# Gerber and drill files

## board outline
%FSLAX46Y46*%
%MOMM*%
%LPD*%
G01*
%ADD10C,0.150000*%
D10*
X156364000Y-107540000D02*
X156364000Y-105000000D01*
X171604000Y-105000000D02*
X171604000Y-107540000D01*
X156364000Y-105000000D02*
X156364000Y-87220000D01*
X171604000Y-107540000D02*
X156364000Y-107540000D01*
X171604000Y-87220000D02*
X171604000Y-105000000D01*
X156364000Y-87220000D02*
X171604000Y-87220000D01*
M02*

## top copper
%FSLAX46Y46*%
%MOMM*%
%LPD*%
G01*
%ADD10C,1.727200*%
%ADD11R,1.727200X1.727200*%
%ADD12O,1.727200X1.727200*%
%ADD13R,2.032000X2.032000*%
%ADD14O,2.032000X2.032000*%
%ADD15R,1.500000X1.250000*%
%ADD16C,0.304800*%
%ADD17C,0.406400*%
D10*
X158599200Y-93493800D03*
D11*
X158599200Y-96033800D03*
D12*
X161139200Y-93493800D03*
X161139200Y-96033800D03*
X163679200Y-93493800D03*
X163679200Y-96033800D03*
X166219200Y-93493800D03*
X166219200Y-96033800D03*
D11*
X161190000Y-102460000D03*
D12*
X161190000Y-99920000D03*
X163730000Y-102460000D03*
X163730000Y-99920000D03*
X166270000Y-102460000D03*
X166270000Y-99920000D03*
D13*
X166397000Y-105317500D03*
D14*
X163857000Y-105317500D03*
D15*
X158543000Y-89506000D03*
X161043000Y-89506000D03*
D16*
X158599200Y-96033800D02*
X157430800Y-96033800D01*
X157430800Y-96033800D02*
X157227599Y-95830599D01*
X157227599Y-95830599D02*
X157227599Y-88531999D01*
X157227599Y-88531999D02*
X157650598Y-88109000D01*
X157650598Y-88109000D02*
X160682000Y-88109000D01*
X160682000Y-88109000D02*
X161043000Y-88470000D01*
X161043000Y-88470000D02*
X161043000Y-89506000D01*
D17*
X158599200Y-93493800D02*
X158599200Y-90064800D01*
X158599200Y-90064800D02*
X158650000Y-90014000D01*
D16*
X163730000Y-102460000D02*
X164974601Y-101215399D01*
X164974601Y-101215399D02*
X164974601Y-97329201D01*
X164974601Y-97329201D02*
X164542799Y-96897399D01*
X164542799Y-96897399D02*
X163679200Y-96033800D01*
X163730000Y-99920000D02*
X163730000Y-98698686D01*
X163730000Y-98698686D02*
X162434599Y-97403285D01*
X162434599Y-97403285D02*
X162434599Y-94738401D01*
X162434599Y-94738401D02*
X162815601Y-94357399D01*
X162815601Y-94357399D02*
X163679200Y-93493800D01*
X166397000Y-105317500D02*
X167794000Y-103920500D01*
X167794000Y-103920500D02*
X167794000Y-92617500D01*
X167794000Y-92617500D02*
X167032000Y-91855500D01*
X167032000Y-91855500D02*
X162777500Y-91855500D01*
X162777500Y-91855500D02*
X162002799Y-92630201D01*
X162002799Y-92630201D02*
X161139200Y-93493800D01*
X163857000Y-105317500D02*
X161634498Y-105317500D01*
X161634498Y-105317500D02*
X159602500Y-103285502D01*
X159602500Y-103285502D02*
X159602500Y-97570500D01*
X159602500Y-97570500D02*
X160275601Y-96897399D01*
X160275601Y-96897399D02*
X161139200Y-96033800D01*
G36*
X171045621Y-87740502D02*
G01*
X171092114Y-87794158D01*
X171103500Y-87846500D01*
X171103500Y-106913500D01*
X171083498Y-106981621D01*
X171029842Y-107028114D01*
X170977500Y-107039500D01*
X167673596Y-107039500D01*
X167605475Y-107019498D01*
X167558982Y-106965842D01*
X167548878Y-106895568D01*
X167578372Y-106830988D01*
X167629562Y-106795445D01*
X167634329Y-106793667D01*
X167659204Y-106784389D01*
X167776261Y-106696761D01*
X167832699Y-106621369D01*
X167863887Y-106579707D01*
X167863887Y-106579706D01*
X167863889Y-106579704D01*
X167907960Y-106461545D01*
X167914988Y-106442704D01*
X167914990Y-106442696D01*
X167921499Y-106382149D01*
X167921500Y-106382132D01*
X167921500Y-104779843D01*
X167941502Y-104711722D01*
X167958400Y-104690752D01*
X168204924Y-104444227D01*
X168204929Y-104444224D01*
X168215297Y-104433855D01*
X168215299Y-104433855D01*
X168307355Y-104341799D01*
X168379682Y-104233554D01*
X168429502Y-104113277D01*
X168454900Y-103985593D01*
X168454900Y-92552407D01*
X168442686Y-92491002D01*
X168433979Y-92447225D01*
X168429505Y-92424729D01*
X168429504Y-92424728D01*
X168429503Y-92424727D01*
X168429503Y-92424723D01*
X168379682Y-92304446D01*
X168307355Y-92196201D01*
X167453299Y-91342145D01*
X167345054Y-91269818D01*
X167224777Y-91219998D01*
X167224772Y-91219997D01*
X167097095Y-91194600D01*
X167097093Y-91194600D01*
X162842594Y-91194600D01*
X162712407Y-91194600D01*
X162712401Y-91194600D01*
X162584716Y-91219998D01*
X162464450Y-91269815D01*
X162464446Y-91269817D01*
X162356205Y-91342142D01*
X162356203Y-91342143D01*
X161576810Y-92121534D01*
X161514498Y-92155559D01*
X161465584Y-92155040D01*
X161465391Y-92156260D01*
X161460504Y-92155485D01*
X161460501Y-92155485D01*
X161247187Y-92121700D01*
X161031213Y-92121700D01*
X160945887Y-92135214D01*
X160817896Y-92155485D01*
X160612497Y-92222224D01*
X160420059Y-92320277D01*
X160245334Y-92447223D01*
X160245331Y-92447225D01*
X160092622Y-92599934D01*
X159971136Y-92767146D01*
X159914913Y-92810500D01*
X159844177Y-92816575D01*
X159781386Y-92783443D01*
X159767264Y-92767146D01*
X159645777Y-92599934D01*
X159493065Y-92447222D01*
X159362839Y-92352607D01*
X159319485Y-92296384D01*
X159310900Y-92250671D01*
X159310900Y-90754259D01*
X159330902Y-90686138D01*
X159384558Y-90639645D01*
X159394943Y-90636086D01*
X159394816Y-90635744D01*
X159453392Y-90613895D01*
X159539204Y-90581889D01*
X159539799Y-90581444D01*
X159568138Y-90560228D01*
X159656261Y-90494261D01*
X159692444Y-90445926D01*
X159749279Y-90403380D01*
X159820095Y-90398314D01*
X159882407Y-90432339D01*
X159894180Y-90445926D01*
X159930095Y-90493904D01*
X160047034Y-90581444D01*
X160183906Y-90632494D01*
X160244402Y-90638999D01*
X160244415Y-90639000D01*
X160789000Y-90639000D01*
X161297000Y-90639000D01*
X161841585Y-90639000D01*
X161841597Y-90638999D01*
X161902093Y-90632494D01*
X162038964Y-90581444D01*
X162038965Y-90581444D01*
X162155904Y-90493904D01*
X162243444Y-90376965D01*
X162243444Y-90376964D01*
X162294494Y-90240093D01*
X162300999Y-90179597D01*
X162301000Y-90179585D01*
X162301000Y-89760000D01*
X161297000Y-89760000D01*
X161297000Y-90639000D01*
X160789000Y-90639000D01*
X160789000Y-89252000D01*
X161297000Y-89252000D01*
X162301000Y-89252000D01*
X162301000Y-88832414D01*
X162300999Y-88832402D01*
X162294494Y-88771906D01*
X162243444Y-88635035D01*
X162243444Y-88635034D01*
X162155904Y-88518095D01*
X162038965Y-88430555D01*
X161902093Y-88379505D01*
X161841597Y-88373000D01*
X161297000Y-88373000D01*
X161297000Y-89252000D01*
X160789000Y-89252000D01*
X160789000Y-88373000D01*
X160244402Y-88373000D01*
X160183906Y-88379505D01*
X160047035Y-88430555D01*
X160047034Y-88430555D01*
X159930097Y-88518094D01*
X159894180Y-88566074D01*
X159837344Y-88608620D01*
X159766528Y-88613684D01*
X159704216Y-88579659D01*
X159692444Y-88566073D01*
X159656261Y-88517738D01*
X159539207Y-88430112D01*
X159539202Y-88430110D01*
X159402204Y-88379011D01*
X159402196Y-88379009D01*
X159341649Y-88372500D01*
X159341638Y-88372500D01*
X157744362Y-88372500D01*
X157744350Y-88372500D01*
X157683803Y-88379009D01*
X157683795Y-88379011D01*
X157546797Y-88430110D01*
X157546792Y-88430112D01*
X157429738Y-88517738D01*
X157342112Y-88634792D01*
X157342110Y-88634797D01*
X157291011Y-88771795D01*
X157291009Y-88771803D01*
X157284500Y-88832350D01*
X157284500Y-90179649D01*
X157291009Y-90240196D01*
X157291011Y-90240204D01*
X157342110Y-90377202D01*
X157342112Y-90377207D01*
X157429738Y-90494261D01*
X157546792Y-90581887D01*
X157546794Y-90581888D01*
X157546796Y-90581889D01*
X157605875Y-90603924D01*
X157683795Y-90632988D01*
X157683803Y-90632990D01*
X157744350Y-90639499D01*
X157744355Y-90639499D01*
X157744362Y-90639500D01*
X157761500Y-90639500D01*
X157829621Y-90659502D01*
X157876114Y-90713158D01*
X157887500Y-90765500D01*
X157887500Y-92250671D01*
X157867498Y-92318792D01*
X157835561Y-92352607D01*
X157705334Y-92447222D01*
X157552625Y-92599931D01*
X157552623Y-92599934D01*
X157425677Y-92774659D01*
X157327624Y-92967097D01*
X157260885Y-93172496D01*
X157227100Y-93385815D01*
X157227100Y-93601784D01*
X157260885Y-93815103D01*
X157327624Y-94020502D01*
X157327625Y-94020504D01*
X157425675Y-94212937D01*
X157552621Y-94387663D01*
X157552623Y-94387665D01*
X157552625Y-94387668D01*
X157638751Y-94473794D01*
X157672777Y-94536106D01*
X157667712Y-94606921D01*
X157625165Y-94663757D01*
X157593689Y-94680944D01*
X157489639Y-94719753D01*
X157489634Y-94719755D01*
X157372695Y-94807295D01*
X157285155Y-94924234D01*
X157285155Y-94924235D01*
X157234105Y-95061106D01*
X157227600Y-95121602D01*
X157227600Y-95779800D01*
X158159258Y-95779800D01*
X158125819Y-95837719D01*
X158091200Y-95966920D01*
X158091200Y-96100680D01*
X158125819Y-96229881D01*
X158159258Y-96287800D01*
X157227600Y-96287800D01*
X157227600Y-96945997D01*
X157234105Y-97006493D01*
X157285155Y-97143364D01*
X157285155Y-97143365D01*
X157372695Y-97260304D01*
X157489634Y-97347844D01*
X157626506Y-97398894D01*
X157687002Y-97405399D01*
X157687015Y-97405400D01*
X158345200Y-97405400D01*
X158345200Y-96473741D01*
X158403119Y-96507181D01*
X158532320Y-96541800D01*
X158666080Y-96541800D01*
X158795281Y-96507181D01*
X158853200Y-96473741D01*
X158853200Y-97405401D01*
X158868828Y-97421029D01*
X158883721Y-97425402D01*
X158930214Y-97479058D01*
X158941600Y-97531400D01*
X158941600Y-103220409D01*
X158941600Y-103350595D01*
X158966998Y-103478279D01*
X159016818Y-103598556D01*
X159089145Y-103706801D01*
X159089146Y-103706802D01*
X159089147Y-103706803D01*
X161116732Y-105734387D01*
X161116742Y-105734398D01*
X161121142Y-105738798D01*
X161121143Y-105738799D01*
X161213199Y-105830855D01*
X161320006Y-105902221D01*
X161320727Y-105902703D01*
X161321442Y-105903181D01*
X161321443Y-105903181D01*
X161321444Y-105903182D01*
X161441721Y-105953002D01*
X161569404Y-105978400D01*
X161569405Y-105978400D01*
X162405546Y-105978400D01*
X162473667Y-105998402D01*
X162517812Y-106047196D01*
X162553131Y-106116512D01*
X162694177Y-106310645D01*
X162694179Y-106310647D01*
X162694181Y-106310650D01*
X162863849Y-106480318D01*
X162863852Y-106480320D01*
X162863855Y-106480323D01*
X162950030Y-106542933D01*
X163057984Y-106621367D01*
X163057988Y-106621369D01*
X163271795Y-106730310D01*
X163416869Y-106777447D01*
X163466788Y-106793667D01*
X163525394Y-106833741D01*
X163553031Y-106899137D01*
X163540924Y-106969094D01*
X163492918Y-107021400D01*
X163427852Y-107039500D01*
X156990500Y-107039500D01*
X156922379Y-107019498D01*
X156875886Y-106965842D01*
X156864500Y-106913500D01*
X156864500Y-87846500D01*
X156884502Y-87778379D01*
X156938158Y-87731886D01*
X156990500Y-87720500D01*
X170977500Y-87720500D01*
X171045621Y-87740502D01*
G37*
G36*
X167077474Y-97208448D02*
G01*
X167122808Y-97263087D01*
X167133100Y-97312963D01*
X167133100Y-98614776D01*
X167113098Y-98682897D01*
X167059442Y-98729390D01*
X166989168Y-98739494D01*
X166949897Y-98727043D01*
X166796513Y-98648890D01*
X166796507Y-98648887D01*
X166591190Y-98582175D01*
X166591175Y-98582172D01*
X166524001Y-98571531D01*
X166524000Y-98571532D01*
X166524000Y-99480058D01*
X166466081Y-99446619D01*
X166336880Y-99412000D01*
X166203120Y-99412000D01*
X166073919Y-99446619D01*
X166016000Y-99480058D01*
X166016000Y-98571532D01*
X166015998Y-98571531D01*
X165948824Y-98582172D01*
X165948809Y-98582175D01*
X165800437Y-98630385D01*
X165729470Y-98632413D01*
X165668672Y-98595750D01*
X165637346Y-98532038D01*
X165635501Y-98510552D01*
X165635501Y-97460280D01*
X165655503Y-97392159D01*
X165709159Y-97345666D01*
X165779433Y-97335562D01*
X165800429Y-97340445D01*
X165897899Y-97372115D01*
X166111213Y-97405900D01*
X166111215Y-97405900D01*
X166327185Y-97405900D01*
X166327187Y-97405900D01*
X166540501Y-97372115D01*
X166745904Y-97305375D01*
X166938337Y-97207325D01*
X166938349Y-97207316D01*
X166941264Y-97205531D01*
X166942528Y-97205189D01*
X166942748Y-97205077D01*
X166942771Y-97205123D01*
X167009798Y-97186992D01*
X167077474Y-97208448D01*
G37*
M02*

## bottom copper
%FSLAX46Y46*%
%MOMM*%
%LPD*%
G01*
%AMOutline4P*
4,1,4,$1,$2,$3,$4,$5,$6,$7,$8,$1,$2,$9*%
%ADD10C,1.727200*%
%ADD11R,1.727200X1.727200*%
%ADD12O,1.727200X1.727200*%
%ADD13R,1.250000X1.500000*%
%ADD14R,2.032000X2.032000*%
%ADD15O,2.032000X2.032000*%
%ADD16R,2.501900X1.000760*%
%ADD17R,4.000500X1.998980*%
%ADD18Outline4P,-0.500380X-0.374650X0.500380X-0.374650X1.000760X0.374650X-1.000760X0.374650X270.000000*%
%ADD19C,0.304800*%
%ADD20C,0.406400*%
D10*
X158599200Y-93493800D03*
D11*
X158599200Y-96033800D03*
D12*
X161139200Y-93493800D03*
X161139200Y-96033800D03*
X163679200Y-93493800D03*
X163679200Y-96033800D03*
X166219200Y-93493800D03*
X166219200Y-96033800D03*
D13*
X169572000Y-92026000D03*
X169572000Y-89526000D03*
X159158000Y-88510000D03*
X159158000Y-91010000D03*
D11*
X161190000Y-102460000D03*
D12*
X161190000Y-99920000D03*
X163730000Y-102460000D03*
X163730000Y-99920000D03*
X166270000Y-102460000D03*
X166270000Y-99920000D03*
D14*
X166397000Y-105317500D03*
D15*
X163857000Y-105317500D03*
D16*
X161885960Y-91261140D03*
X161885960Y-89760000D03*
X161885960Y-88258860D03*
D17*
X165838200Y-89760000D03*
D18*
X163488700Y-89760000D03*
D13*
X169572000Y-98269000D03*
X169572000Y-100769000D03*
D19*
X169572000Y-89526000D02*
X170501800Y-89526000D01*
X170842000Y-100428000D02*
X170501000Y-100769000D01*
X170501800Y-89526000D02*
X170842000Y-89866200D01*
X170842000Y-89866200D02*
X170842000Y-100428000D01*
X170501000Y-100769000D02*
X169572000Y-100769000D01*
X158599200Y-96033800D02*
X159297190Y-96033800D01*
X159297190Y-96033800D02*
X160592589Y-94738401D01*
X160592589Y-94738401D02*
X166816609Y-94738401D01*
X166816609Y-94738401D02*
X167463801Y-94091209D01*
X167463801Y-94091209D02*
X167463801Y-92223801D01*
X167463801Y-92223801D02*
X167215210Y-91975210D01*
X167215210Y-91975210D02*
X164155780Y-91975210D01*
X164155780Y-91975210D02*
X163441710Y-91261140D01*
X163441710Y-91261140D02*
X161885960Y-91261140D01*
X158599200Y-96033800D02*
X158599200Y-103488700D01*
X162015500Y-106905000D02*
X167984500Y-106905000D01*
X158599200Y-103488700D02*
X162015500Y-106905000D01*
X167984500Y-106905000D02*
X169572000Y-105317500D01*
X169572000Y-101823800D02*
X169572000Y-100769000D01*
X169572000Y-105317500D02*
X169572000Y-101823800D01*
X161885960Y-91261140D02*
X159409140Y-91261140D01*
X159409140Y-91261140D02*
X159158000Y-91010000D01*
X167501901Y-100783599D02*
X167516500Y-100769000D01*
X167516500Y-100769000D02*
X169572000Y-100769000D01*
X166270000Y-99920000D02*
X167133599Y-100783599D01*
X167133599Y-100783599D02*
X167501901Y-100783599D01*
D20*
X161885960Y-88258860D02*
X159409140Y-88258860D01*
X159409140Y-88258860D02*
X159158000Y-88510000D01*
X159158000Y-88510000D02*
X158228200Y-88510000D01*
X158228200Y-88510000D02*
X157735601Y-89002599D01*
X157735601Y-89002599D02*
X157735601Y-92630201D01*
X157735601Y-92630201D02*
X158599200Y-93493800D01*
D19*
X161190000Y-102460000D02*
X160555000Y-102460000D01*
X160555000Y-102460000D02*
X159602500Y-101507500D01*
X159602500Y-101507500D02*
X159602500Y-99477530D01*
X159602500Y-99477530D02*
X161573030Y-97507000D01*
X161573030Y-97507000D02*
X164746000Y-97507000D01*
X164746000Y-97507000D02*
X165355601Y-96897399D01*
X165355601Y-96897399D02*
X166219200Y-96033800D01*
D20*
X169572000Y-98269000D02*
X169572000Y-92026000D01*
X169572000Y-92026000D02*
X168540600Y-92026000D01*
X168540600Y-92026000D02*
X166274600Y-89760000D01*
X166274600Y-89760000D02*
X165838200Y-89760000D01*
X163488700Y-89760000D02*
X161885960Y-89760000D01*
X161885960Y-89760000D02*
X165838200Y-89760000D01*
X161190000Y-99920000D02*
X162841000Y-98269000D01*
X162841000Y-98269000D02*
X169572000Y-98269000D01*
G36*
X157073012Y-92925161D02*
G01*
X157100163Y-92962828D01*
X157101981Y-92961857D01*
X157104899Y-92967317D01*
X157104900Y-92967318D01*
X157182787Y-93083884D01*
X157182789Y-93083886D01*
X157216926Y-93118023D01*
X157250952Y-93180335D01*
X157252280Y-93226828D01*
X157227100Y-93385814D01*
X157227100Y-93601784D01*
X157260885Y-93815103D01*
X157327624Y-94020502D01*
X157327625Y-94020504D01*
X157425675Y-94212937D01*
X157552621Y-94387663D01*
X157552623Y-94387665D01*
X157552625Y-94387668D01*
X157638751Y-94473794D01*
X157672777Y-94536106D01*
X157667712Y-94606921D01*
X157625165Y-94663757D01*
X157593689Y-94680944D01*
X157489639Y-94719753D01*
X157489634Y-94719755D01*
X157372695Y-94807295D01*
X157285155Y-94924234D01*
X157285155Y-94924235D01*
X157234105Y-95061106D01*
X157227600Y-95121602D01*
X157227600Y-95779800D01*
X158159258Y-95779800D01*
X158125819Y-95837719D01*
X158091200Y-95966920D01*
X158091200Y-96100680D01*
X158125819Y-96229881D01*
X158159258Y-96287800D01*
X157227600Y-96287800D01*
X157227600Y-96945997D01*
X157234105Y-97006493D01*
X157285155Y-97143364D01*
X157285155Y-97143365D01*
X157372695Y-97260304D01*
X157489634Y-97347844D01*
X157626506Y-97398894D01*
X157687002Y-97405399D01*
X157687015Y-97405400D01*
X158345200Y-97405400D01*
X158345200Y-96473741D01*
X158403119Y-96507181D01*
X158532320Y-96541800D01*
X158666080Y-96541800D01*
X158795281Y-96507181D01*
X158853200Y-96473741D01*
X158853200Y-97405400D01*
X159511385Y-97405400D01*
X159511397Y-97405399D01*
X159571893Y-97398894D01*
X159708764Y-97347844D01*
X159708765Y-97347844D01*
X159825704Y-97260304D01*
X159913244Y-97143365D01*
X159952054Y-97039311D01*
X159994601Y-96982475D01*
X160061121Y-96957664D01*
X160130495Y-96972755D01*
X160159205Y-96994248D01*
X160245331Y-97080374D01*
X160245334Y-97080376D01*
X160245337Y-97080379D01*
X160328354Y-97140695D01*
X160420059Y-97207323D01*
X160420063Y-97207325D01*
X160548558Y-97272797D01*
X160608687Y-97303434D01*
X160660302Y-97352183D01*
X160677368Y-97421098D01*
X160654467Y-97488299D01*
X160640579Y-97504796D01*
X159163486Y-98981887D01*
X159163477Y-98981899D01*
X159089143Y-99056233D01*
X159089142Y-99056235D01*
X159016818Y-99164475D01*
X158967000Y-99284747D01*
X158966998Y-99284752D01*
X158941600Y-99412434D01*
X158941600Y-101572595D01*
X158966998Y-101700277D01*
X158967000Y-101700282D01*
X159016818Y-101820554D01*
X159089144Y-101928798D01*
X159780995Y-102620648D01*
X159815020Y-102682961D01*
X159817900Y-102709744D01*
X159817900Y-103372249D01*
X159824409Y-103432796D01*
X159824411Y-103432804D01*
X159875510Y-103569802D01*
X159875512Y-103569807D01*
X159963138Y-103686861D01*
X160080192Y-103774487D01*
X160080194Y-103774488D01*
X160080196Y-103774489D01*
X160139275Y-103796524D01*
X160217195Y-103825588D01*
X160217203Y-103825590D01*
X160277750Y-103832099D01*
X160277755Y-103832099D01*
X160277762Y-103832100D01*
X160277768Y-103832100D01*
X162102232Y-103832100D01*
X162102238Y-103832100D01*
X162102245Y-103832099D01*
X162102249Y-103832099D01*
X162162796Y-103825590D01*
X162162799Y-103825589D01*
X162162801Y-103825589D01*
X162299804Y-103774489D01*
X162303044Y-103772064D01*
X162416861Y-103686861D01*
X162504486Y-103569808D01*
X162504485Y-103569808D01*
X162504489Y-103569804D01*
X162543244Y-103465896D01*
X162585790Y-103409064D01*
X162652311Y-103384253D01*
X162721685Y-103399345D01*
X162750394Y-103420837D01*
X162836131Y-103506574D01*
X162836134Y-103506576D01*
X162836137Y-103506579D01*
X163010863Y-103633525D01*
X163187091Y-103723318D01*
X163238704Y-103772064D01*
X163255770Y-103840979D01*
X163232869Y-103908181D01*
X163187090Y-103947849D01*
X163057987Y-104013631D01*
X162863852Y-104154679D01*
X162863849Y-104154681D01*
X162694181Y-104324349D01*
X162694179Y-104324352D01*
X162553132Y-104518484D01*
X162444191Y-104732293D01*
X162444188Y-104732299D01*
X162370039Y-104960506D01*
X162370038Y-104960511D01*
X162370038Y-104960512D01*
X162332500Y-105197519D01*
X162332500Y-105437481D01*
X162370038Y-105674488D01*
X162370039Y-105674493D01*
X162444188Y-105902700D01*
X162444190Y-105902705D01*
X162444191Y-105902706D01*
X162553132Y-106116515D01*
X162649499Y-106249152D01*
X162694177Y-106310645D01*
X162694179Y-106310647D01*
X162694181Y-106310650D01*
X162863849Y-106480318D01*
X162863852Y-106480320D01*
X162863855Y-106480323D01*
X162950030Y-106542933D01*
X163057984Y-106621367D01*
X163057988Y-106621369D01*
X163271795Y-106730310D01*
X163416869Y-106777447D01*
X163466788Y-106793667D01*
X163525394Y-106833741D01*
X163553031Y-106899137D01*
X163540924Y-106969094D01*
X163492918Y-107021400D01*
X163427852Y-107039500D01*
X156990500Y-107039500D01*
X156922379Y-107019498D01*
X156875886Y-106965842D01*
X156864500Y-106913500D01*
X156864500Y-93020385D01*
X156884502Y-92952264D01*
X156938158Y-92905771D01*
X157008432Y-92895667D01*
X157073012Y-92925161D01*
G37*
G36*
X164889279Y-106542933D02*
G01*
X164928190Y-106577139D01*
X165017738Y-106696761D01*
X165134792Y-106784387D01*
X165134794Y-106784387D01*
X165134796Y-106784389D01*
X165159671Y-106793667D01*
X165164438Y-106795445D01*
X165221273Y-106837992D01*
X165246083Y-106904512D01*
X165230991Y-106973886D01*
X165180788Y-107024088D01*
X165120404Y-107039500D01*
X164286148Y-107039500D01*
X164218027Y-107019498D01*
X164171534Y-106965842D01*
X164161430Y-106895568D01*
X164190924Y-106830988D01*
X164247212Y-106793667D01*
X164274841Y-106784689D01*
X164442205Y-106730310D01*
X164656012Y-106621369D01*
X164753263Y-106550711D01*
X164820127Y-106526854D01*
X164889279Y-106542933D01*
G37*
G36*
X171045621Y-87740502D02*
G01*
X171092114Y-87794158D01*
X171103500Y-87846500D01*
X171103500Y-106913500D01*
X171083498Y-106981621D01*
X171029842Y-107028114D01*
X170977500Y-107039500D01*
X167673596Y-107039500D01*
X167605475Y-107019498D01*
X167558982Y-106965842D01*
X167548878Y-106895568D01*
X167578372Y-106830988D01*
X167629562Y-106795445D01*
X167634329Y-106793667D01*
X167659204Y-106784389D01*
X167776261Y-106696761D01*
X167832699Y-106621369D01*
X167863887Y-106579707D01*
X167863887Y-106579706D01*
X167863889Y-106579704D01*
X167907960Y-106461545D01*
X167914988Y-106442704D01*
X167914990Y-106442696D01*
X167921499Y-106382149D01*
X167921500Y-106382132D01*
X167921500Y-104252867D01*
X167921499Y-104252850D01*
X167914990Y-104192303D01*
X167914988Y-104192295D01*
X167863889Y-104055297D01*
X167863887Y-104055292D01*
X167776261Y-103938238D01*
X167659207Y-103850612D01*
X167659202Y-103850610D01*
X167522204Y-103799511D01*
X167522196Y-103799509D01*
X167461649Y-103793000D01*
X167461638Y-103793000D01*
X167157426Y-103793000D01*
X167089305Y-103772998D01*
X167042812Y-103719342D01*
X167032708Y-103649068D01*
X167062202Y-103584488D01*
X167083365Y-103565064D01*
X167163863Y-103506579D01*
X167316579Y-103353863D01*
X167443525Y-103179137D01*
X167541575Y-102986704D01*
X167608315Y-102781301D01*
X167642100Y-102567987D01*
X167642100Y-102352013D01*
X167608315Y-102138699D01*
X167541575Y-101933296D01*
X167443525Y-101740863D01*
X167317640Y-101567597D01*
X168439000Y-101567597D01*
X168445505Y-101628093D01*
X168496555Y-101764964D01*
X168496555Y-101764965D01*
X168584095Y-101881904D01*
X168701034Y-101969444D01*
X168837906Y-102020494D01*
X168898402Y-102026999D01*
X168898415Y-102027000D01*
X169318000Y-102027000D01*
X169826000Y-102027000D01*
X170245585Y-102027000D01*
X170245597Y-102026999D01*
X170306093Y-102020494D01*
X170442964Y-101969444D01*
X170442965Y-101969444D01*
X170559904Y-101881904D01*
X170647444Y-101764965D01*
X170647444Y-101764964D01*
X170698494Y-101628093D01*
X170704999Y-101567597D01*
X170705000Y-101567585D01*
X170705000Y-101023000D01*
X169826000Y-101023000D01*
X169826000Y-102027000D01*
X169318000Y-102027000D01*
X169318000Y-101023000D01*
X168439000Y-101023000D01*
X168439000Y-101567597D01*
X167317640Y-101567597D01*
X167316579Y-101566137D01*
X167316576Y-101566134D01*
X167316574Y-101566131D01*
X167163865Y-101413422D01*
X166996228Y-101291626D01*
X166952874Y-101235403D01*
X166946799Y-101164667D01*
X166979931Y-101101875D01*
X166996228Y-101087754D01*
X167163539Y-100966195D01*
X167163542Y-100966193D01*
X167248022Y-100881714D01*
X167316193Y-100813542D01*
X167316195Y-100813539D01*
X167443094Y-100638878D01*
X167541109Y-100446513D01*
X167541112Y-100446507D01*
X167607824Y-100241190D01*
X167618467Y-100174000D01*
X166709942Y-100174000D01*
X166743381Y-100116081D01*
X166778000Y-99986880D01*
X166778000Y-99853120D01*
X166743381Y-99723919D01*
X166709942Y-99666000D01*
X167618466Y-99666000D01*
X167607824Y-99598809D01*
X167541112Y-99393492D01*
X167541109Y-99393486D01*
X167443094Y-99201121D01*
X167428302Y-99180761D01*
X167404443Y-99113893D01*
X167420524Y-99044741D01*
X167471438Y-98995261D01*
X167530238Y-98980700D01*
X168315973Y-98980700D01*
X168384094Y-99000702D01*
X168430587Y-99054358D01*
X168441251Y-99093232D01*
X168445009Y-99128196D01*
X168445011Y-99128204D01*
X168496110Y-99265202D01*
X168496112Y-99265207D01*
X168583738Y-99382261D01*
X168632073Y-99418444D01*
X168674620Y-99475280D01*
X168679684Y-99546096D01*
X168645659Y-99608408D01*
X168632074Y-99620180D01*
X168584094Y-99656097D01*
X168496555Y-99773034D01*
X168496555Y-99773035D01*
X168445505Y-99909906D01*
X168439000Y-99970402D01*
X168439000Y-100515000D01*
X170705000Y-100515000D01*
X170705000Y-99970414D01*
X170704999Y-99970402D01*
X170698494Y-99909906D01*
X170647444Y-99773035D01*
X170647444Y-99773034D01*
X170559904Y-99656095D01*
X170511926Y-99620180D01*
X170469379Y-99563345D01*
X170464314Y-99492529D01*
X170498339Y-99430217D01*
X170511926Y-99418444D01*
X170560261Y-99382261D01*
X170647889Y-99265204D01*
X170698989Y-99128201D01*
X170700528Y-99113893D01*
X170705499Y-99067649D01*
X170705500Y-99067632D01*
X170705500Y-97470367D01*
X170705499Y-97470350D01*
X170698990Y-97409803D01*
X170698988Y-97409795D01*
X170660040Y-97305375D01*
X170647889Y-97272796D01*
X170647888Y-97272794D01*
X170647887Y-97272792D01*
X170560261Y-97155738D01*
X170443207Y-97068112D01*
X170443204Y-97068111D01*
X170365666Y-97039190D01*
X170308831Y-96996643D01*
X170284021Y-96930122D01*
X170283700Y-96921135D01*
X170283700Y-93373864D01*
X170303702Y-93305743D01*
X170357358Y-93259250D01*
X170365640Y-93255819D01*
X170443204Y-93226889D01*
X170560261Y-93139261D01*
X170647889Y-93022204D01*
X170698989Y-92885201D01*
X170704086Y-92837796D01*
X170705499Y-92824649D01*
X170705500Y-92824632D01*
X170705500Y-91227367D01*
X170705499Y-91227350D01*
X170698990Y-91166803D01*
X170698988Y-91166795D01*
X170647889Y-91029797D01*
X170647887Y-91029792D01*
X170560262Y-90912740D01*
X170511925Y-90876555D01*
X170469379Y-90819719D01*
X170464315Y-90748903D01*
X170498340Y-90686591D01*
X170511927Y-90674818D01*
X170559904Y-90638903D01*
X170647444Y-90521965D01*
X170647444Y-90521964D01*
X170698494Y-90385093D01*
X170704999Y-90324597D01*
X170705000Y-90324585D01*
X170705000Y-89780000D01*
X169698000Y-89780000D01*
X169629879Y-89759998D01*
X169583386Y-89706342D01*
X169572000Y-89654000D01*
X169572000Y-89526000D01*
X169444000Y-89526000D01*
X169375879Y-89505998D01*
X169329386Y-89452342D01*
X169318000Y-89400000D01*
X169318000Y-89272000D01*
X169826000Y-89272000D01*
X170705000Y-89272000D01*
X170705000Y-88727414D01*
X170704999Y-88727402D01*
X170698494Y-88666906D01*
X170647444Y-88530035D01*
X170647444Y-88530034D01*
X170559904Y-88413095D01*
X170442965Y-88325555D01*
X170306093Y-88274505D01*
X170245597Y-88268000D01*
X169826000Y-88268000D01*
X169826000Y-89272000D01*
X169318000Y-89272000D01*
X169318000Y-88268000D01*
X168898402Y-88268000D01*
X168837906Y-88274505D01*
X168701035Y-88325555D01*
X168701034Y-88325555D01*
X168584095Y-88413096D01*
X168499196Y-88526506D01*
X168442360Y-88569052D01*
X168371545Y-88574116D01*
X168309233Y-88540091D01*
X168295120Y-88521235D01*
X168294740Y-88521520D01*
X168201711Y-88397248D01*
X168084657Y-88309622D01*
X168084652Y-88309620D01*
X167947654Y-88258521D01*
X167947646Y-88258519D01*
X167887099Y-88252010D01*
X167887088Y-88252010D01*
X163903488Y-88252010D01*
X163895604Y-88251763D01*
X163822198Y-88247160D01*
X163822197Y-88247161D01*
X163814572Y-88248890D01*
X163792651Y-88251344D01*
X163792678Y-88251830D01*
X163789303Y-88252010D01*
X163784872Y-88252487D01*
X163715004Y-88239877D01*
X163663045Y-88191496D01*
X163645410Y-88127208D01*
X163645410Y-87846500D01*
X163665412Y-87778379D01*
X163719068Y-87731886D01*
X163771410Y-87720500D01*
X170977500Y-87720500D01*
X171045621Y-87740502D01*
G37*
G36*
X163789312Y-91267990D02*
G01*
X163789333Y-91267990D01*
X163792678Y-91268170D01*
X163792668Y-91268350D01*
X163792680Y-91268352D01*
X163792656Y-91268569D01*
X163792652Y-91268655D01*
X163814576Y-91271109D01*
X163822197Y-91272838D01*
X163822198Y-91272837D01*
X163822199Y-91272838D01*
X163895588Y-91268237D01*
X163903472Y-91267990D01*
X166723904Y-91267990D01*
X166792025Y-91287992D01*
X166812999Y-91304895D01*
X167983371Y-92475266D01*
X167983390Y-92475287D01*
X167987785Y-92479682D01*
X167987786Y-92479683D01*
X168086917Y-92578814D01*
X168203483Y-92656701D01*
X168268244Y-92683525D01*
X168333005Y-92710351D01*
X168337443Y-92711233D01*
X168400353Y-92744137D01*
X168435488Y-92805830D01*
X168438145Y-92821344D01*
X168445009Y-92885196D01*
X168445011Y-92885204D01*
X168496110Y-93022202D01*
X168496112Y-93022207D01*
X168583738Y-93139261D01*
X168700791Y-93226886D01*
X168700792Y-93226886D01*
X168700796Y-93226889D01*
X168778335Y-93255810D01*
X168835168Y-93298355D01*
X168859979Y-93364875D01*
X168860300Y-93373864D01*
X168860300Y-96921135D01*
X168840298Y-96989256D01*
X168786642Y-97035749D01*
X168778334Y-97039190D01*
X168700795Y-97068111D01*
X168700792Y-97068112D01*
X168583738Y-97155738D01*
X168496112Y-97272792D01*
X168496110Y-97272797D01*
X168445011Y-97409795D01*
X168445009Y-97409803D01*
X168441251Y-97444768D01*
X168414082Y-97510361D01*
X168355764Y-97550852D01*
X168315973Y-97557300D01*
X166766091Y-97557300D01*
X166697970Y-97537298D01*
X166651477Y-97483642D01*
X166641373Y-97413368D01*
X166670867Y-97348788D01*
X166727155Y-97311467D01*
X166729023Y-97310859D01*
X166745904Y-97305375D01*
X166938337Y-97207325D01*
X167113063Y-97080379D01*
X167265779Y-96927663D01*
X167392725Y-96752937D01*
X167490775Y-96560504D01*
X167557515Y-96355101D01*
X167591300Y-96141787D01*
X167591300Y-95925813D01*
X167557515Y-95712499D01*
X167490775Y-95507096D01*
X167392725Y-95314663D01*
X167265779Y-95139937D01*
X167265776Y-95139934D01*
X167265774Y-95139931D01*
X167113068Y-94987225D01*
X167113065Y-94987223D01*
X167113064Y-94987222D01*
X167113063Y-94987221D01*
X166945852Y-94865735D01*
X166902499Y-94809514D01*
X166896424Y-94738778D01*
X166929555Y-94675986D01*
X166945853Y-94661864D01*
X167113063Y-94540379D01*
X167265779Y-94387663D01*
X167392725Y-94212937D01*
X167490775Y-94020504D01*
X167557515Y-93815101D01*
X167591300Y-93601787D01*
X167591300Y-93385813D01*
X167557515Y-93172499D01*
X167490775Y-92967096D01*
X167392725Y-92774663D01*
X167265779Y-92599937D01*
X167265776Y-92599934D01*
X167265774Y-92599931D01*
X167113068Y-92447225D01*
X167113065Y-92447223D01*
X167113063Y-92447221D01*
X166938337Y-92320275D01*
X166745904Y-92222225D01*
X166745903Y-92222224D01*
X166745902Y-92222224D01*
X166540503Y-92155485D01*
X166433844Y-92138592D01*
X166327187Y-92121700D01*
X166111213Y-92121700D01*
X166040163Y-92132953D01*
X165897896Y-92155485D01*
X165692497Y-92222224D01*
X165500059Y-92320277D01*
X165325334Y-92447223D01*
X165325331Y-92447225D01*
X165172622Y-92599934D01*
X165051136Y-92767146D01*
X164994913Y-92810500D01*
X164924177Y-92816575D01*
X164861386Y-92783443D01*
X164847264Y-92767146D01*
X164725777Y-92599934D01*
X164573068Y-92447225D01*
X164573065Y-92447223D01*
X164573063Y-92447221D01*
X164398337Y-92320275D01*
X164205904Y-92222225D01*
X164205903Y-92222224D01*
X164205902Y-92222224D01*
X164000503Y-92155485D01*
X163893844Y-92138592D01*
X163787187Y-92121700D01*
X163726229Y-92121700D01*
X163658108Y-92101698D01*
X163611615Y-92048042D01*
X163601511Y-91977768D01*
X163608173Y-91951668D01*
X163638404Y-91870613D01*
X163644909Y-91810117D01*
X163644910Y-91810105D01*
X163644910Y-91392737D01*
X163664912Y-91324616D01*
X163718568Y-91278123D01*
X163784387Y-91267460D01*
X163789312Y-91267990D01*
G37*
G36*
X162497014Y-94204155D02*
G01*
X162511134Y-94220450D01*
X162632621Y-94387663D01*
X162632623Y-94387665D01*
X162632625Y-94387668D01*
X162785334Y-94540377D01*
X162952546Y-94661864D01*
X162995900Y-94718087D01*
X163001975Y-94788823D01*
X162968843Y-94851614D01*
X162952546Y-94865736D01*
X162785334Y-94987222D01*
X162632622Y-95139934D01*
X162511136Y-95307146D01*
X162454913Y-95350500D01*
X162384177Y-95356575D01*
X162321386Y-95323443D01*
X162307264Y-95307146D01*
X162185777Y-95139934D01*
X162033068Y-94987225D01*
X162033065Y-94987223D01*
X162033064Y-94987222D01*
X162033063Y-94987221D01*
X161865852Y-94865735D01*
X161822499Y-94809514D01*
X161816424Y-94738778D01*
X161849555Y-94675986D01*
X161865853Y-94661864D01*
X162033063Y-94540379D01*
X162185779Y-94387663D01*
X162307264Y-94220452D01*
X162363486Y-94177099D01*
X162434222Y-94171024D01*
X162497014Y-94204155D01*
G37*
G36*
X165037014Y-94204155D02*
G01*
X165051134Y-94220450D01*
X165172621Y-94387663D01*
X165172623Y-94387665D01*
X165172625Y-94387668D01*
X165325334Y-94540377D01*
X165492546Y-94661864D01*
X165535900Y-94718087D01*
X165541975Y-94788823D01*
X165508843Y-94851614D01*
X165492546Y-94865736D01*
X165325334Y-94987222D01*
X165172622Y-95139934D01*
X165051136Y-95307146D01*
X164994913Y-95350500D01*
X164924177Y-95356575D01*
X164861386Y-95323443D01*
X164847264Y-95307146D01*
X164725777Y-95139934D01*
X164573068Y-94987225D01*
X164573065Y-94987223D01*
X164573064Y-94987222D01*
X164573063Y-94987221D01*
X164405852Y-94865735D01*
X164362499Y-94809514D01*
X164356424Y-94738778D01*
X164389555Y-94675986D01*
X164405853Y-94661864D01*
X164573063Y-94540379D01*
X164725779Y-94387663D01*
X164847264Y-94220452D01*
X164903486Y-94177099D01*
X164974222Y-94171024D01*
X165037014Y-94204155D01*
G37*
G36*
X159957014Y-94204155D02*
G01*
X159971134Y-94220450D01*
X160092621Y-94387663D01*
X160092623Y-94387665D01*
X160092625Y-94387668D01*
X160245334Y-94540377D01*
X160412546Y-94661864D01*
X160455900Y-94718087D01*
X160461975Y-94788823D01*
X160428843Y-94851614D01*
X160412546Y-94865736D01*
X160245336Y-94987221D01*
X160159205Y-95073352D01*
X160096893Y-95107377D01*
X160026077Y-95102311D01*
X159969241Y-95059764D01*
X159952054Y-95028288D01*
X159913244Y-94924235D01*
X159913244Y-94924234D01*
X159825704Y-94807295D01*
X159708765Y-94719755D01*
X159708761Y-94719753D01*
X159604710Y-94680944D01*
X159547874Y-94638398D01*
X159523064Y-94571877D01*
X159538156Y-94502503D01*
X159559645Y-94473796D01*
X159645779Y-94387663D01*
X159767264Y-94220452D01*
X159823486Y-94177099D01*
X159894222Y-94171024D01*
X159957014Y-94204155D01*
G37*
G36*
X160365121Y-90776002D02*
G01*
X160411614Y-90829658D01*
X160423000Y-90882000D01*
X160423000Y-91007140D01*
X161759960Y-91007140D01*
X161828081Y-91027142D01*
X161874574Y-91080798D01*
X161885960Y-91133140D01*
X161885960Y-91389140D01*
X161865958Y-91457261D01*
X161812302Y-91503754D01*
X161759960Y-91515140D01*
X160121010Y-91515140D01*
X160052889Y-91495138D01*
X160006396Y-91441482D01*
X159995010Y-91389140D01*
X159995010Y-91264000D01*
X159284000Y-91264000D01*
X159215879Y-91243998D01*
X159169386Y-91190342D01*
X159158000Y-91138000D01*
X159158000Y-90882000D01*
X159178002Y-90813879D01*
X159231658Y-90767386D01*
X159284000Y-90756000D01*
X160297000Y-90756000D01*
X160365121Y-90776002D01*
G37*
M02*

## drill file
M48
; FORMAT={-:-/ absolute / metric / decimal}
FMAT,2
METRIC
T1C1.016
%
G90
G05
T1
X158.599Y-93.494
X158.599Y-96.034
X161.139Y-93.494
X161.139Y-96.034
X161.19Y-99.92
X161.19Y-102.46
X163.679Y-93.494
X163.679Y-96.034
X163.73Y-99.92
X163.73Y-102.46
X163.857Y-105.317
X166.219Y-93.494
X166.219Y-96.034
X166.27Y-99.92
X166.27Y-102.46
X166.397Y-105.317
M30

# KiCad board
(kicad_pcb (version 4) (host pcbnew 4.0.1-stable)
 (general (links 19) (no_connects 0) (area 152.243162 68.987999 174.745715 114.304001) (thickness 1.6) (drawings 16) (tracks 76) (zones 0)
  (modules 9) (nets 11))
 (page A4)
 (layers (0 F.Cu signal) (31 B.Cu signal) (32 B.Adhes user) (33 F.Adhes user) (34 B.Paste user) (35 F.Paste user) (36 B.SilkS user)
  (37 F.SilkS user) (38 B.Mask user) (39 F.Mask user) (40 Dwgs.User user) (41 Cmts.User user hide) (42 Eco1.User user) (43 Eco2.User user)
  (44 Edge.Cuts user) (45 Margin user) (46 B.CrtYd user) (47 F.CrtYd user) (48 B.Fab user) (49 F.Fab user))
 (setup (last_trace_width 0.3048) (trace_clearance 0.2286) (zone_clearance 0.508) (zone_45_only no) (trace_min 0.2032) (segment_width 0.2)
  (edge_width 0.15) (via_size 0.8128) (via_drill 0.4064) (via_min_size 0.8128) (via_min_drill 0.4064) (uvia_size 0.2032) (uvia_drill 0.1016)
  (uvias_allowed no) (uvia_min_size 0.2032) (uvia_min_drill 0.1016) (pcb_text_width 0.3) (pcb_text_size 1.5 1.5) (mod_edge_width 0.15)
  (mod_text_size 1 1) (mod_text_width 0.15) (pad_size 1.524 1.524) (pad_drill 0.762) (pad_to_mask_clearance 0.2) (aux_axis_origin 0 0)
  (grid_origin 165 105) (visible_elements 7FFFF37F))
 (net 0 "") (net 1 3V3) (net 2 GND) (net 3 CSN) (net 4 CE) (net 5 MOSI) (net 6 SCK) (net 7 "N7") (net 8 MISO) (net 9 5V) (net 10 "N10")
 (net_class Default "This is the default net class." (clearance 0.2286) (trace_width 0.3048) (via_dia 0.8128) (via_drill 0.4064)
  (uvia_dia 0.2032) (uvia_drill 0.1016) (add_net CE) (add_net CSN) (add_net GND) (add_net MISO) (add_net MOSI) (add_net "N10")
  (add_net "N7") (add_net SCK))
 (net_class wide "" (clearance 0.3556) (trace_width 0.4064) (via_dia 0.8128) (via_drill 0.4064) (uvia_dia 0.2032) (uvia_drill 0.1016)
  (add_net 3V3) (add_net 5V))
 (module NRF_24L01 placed (layer F.Cu) (at 162.46 93.57)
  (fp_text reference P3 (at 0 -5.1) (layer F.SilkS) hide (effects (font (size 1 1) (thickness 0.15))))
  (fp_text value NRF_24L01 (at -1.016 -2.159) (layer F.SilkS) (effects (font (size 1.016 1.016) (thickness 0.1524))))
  (pad 2 thru_hole circle (at -3.8608 -0.0762) (size 1.7272 1.7272) (drill 1.016) (layers *.Cu *.Mask F.SilkS) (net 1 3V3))
  (pad 1 thru_hole rect (at -3.8608 2.4638) (size 1.7272 1.7272) (drill 1.016) (layers *.Cu *.Mask F.SilkS) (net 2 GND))
  (pad 4 thru_hole oval (at -1.3208 -0.0762) (size 1.7272 1.7272) (drill 1.016) (layers *.Cu *.Mask F.SilkS) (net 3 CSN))
  (pad 3 thru_hole oval (at -1.3208 2.4638) (size 1.7272 1.7272) (drill 1.016) (layers *.Cu *.Mask F.SilkS) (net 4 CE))
  (pad 6 thru_hole oval (at 1.2192 -0.0762) (size 1.7272 1.7272) (drill 1.016) (layers *.Cu *.Mask F.SilkS) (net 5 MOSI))
  (pad 5 thru_hole oval (at 1.2192 2.4638) (size 1.7272 1.7272) (drill 1.016) (layers *.Cu *.Mask F.SilkS) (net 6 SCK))
  (pad 8 thru_hole oval (at 3.7592 -0.0762) (size 1.7272 1.7272) (drill 1.016) (layers *.Cu *.Mask F.SilkS) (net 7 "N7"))
  (pad 7 thru_hole oval (at 3.7592 2.4638) (size 1.7272 1.7272) (drill 1.016) (layers *.Cu *.Mask F.SilkS) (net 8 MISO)))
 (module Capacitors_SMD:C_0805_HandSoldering (layer B.Cu) (at 169.572 90.776 90)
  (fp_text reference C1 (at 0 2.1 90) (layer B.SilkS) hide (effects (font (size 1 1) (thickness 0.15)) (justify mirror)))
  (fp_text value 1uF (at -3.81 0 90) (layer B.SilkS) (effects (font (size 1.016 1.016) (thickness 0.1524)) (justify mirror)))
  (pad 1 smd rect (at -1.25 0 90) (size 1.5 1.25) (layers B.Cu B.Paste B.Mask) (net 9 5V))
  (pad 2 smd rect (at 1.25 0 90) (size 1.5 1.25) (layers B.Cu B.Paste B.Mask) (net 2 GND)))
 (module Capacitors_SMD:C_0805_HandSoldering (layer B.Cu) (at 159.158 89.76 270)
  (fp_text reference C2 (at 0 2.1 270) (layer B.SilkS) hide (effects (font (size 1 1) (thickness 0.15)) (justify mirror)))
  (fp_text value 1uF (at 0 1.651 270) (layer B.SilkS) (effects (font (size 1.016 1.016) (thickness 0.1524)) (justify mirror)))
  (pad 1 smd rect (at -1.25 0 270) (size 1.5 1.25) (layers B.Cu B.Paste B.Mask) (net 1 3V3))
  (pad 2 smd rect (at 1.25 0 270) (size 1.5 1.25) (layers B.Cu B.Paste B.Mask) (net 2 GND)))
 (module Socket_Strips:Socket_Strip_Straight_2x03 (layer B.Cu) (at 161.19 102.46)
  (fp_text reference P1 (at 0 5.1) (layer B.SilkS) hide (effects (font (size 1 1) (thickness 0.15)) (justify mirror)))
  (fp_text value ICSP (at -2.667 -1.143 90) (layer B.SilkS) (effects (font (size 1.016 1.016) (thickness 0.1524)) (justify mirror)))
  (pad 1 thru_hole rect (at 0 0) (size 1.7272 1.7272) (drill 1.016) (layers *.Cu *.Mask B.SilkS) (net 8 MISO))
  (pad 2 thru_hole oval (at 0 -2.54) (size 1.7272 1.7272) (drill 1.016) (layers *.Cu *.Mask B.SilkS) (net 9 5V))
  (pad 3 thru_hole oval (at 2.54 0) (size 1.7272 1.7272) (drill 1.016) (layers *.Cu *.Mask B.SilkS) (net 6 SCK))
  (pad 4 thru_hole oval (at 2.54 -2.54) (size 1.7272 1.7272) (drill 1.016) (layers *.Cu *.Mask B.SilkS) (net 5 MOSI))
  (pad 5 thru_hole oval (at 5.08 0) (size 1.7272 1.7272) (drill 1.016) (layers *.Cu *.Mask B.SilkS) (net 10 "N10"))
  (pad 6 thru_hole oval (at 5.08 -2.54) (size 1.7272 1.7272) (drill 1.016) (layers *.Cu *.Mask B.SilkS) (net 2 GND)))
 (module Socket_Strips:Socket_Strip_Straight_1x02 (layer F.Cu) (at 166.397 105.3175 180)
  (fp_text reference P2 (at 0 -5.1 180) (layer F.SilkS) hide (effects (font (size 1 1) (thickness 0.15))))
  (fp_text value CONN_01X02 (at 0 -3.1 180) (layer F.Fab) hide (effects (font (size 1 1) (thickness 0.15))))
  (pad 1 thru_hole rect (at 0 0 180) (size 2.032 2.032) (drill 1.016) (layers *.Cu *.Mask F.SilkS) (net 3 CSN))
  (pad 2 thru_hole oval (at 2.54 0 180) (size 2.032 2.032) (drill 1.016) (layers *.Cu *.Mask F.SilkS) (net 4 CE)))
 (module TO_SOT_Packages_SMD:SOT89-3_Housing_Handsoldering (layer B.Cu) (at 164.238 89.76 90)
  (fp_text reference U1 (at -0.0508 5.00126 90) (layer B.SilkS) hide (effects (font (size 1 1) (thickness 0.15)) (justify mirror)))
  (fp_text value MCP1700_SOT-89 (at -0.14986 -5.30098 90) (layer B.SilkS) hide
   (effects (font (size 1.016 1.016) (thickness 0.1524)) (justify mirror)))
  (pad 1 smd rect (at -1.50114 -2.35204 90) (size 1.00076 2.5019) (layers B.Cu B.Paste B.Mask) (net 2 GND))
  (pad 2 smd rect (at 0 -2.35204 90) (size 1.00076 2.5019) (layers B.Cu B.Paste B.Mask) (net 9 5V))
  (pad 3 smd rect (at 1.50114 -2.35204 90) (size 1.00076 2.5019) (layers B.Cu B.Paste B.Mask) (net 1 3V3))
  (pad 2 smd rect (at 0 1.6002 90) (size 1.99898 4.0005) (layers B.Cu B.Paste B.Mask) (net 9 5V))
  (pad 2 smd trapezoid (at 0 -0.7493 270) (size 1.50114 0.7493) (rect_delta 0 -0.50038) (layers B.Cu B.Paste B.Mask) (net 9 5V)))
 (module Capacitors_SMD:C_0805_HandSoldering (layer F.Cu) (at 159.793 89.506)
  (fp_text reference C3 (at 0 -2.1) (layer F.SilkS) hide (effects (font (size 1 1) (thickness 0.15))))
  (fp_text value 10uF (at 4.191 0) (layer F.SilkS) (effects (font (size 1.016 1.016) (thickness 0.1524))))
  (pad 1 smd rect (at -1.25 0) (size 1.5 1.25) (layers F.Cu F.Paste F.Mask) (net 1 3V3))
  (pad 2 smd rect (at 1.25 0) (size 1.5 1.25) (layers F.Cu F.Paste F.Mask) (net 2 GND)))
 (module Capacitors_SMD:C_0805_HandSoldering (layer B.Cu) (at 169.572 99.519 270)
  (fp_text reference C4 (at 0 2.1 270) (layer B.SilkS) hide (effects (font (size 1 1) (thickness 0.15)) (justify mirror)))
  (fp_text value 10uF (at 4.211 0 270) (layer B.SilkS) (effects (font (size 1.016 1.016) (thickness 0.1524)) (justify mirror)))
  (pad 1 smd rect (at -1.25 0 270) (size 1.5 1.25) (layers B.Cu B.Paste B.Mask) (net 9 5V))
  (pad 2 smd rect (at 1.25 0 270) (size 1.5 1.25) (layers B.Cu B.Paste B.Mask) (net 2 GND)))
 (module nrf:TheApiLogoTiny (layer F.Cu) (at 158.269 102.206)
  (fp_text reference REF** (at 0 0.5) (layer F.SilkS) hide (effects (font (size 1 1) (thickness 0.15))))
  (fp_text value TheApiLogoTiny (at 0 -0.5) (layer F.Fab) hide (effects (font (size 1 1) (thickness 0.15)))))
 (gr_line (start 156.364 107.54) (end 156.364 105) (angle 90) (layer Edge.Cuts) (width 0.15))
 (gr_line (start 171.604 105) (end 171.604 107.54) (angle 90) (layer Edge.Cuts) (width 0.15))
 (gr_line (start 156.364 105) (end 156.364 87.22) (angle 90) (layer Edge.Cuts) (width 0.15))
 (gr_line (start 171.604 107.54) (end 156.364 107.54) (angle 90) (layer Edge.Cuts) (width 0.15))
 (gr_line (start 171.604 87.22) (end 171.604 105) (angle 90) (layer Edge.Cuts) (width 0.15))
 (gr_line (start 156.364 87.22) (end 171.604 87.22) (angle 90) (layer Edge.Cuts) (width 0.15))
 (segment (start 158.5992 96.0338) (end 157.4308 96.0338) (width 0.3048) (layer F.Cu) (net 2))
 (segment (start 157.4308 96.0338) (end 157.227599 95.830599) (width 0.3048) (layer F.Cu) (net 2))
 (segment (start 157.227599 95.830599) (end 157.227599 88.531999) (width 0.3048) (layer F.Cu) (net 2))
 (segment (start 157.227599 88.531999) (end 157.650598 88.109) (width 0.3048) (layer F.Cu) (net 2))
 (segment (start 157.650598 88.109) (end 160.682 88.109) (width 0.3048) (layer F.Cu) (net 2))
 (segment (start 160.682 88.109) (end 161.043 88.47) (width 0.3048) (layer F.Cu) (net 2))
 (segment (start 161.043 88.47) (end 161.043 89.506) (width 0.3048) (layer F.Cu) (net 2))
 (segment (start 169.572 89.526) (end 170.5018 89.526) (width 0.3048) (layer B.Cu) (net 2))
 (segment (start 170.842 100.428) (end 170.501 100.769) (width 0.3048) (layer B.Cu) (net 2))
 (segment (start 170.5018 89.526) (end 170.842 89.8662) (width 0.3048) (layer B.Cu) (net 2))
 (segment (start 170.842 89.8662) (end 170.842 100.428) (width 0.3048) (layer B.Cu) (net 2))
 (segment (start 170.501 100.769) (end 169.572 100.769) (width 0.3048) (layer B.Cu) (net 2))
 (segment (start 158.5992 96.0338) (end 159.29719 96.0338) (width 0.3048) (layer B.Cu) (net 2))
 (segment (start 159.29719 96.0338) (end 160.592589 94.738401) (width 0.3048) (layer B.Cu) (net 2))
 (segment (start 160.592589 94.738401) (end 166.816609 94.738401) (width 0.3048) (layer B.Cu) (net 2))
 (segment (start 166.816609 94.738401) (end 167.463801 94.091209) (width 0.3048) (layer B.Cu) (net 2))
 (segment (start 167.463801 94.091209) (end 167.463801 92.223801) (width 0.3048) (layer B.Cu) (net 2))
 (segment (start 167.463801 92.223801) (end 167.21521 91.97521) (width 0.3048) (layer B.Cu) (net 2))
 (segment (start 167.21521 91.97521) (end 164.15578 91.97521) (width 0.3048) (layer B.Cu) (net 2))
 (segment (start 164.15578 91.97521) (end 163.44171 91.26114) (width 0.3048) (layer B.Cu) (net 2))
 (segment (start 163.44171 91.26114) (end 161.88596 91.26114) (width 0.3048) (layer B.Cu) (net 2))
 (segment (start 158.5992 96.0338) (end 158.5992 103.4887) (width 0.3048) (layer B.Cu) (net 2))
 (segment (start 162.0155 106.905) (end 167.9845 106.905) (width 0.3048) (layer B.Cu) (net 2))
 (segment (start 158.5992 103.4887) (end 162.0155 106.905) (width 0.3048) (layer B.Cu) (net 2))
 (segment (start 167.9845 106.905) (end 169.572 105.3175) (width 0.3048) (layer B.Cu) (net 2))
 (segment (start 169.572 101.8238) (end 169.572 100.769) (width 0.3048) (layer B.Cu) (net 2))
 (segment (start 169.572 105.3175) (end 169.572 101.8238) (width 0.3048) (layer B.Cu) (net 2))
 (segment (start 161.88596 91.26114) (end 159.40914 91.26114) (width 0.3048) (layer B.Cu) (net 2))
 (segment (start 159.40914 91.26114) (end 159.158 91.01) (width 0.3048) (layer B.Cu) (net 2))
 (segment (start 167.501901 100.783599) (end 167.5165 100.769) (width 0.3048) (layer B.Cu) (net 2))
 (segment (start 167.5165 100.769) (end 169.572 100.769) (width 0.3048) (layer B.Cu) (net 2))
 (segment (start 166.27 99.92) (end 167.133599 100.783599) (width 0.3048) (layer B.Cu) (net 2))
 (segment (start 167.133599 100.783599) (end 167.501901 100.783599) (width 0.3048) (layer B.Cu) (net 2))
 (segment (start 158.5992 93.4938) (end 158.5992 90.0648) (width 0.4064) (layer F.Cu) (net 1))
 (segment (start 158.5992 90.0648) (end 158.65 90.014) (width 0.4064) (layer F.Cu) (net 1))
 (segment (start 161.88596 88.25886) (end 159.40914 88.25886) (width 0.4064) (layer B.Cu) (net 1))
 (segment (start 159.40914 88.25886) (end 159.158 88.51) (width 0.4064) (layer B.Cu) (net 1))
 (segment (start 159.158 88.51) (end 158.2282 88.51) (width 0.4064) (layer B.Cu) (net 1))
 (segment (start 158.2282 88.51) (end 157.735601 89.002599) (width 0.4064) (layer B.Cu) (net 1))
 (segment (start 157.735601 89.002599) (end 157.735601 92.630201) (width 0.4064) (layer B.Cu) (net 1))
 (segment (start 157.735601 92.630201) (end 158.5992 93.4938) (width 0.4064) (layer B.Cu) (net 1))
 (segment (start 163.73 102.46) (end 164.974601 101.215399) (width 0.3048) (layer F.Cu) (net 6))
 (segment (start 164.974601 101.215399) (end 164.974601 97.329201) (width 0.3048) (layer F.Cu) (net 6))
 (segment (start 164.974601 97.329201) (end 164.542799 96.897399) (width 0.3048) (layer F.Cu) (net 6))
 (segment (start 164.542799 96.897399) (end 163.6792 96.0338) (width 0.3048) (layer F.Cu) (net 6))
 (segment (start 163.73 99.92) (end 163.73 98.698686) (width 0.3048) (layer F.Cu) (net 5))
 (segment (start 163.73 98.698686) (end 162.434599 97.403285) (width 0.3048) (layer F.Cu) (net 5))
 (segment (start 162.434599 97.403285) (end 162.434599 94.738401) (width 0.3048) (layer F.Cu) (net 5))
 (segment (start 162.434599 94.738401) (end 162.815601 94.357399) (width 0.3048) (layer F.Cu) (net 5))
 (segment (start 162.815601 94.357399) (end 163.6792 93.4938) (width 0.3048) (layer F.Cu) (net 5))
 (segment (start 161.19 102.46) (end 160.555 102.46) (width 0.3048) (layer B.Cu) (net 8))
 (segment (start 160.555 102.46) (end 159.6025 101.5075) (width 0.3048) (layer B.Cu) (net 8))
 (segment (start 159.6025 101.5075) (end 159.6025 99.47753) (width 0.3048) (layer B.Cu) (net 8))
 (segment (start 159.6025 99.47753) (end 161.57303 97.507) (width 0.3048) (layer B.Cu) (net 8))
 (segment (start 161.57303 97.507) (end 164.746 97.507) (width 0.3048) (layer B.Cu) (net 8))
 (segment (start 164.746 97.507) (end 165.355601 96.897399) (width 0.3048) (layer B.Cu) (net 8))
 (segment (start 165.355601 96.897399) (end 166.2192 96.0338) (width 0.3048) (layer B.Cu) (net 8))
 (segment (start 169.572 98.269) (end 169.572 92.026) (width 0.4064) (layer B.Cu) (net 9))
 (segment (start 169.572 92.026) (end 168.5406 92.026) (width 0.4064) (layer B.Cu) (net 9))
 (segment (start 168.5406 92.026) (end 166.2746 89.76) (width 0.4064) (layer B.Cu) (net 9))
 (segment (start 166.2746 89.76) (end 165.8382 89.76) (width 0.4064) (layer B.Cu) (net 9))
 (segment (start 163.4887 89.76) (end 161.88596 89.76) (width 0.4064) (layer B.Cu) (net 9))
 (segment (start 161.88596 89.76) (end 165.8382 89.76) (width 0.4064) (layer B.Cu) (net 9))
 (segment (start 161.19 99.92) (end 162.841 98.269) (width 0.4064) (layer B.Cu) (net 9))
 (segment (start 162.841 98.269) (end 169.572 98.269) (width 0.4064) (layer B.Cu) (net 9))
 (segment (start 166.397 105.3175) (end 167.794 103.9205) (width 0.3048) (layer F.Cu) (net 3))
 (segment (start 167.794 103.9205) (end 167.794 92.6175) (width 0.3048) (layer F.Cu) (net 3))
 (segment (start 167.794 92.6175) (end 167.032 91.8555) (width 0.3048) (layer F.Cu) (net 3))
 (segment (start 167.032 91.8555) (end 162.7775 91.8555) (width 0.3048) (layer F.Cu) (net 3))
 (segment (start 162.7775 91.8555) (end 162.002799 92.630201) (width 0.3048) (layer F.Cu) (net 3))
 (segment (start 162.002799 92.630201) (end 161.1392 93.4938) (width 0.3048) (layer F.Cu) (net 3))
 (segment (start 163.857 105.3175) (end 161.634498 105.3175) (width 0.3048) (layer F.Cu) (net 4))
 (segment (start 161.634498 105.3175) (end 159.6025 103.285502) (width 0.3048) (layer F.Cu) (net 4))
 (segment (start 159.6025 103.285502) (end 159.6025 97.5705) (width 0.3048) (layer F.Cu) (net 4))
 (segment (start 159.6025 97.5705) (end 160.275601 96.897399) (width 0.3048) (layer F.Cu) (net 4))
 (segment (start 160.275601 96.897399) (end 161.1392 96.0338) (width 0.3048) (layer F.Cu) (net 4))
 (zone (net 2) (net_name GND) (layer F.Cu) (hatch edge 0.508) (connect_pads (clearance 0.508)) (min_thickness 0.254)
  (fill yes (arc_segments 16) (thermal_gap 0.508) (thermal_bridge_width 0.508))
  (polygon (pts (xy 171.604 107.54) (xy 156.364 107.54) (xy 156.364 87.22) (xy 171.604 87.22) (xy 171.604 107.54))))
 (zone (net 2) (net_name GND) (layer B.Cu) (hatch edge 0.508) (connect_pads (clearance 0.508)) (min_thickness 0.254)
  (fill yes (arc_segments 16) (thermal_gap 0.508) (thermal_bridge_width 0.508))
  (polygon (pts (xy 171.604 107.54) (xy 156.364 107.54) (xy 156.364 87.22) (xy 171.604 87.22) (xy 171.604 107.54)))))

